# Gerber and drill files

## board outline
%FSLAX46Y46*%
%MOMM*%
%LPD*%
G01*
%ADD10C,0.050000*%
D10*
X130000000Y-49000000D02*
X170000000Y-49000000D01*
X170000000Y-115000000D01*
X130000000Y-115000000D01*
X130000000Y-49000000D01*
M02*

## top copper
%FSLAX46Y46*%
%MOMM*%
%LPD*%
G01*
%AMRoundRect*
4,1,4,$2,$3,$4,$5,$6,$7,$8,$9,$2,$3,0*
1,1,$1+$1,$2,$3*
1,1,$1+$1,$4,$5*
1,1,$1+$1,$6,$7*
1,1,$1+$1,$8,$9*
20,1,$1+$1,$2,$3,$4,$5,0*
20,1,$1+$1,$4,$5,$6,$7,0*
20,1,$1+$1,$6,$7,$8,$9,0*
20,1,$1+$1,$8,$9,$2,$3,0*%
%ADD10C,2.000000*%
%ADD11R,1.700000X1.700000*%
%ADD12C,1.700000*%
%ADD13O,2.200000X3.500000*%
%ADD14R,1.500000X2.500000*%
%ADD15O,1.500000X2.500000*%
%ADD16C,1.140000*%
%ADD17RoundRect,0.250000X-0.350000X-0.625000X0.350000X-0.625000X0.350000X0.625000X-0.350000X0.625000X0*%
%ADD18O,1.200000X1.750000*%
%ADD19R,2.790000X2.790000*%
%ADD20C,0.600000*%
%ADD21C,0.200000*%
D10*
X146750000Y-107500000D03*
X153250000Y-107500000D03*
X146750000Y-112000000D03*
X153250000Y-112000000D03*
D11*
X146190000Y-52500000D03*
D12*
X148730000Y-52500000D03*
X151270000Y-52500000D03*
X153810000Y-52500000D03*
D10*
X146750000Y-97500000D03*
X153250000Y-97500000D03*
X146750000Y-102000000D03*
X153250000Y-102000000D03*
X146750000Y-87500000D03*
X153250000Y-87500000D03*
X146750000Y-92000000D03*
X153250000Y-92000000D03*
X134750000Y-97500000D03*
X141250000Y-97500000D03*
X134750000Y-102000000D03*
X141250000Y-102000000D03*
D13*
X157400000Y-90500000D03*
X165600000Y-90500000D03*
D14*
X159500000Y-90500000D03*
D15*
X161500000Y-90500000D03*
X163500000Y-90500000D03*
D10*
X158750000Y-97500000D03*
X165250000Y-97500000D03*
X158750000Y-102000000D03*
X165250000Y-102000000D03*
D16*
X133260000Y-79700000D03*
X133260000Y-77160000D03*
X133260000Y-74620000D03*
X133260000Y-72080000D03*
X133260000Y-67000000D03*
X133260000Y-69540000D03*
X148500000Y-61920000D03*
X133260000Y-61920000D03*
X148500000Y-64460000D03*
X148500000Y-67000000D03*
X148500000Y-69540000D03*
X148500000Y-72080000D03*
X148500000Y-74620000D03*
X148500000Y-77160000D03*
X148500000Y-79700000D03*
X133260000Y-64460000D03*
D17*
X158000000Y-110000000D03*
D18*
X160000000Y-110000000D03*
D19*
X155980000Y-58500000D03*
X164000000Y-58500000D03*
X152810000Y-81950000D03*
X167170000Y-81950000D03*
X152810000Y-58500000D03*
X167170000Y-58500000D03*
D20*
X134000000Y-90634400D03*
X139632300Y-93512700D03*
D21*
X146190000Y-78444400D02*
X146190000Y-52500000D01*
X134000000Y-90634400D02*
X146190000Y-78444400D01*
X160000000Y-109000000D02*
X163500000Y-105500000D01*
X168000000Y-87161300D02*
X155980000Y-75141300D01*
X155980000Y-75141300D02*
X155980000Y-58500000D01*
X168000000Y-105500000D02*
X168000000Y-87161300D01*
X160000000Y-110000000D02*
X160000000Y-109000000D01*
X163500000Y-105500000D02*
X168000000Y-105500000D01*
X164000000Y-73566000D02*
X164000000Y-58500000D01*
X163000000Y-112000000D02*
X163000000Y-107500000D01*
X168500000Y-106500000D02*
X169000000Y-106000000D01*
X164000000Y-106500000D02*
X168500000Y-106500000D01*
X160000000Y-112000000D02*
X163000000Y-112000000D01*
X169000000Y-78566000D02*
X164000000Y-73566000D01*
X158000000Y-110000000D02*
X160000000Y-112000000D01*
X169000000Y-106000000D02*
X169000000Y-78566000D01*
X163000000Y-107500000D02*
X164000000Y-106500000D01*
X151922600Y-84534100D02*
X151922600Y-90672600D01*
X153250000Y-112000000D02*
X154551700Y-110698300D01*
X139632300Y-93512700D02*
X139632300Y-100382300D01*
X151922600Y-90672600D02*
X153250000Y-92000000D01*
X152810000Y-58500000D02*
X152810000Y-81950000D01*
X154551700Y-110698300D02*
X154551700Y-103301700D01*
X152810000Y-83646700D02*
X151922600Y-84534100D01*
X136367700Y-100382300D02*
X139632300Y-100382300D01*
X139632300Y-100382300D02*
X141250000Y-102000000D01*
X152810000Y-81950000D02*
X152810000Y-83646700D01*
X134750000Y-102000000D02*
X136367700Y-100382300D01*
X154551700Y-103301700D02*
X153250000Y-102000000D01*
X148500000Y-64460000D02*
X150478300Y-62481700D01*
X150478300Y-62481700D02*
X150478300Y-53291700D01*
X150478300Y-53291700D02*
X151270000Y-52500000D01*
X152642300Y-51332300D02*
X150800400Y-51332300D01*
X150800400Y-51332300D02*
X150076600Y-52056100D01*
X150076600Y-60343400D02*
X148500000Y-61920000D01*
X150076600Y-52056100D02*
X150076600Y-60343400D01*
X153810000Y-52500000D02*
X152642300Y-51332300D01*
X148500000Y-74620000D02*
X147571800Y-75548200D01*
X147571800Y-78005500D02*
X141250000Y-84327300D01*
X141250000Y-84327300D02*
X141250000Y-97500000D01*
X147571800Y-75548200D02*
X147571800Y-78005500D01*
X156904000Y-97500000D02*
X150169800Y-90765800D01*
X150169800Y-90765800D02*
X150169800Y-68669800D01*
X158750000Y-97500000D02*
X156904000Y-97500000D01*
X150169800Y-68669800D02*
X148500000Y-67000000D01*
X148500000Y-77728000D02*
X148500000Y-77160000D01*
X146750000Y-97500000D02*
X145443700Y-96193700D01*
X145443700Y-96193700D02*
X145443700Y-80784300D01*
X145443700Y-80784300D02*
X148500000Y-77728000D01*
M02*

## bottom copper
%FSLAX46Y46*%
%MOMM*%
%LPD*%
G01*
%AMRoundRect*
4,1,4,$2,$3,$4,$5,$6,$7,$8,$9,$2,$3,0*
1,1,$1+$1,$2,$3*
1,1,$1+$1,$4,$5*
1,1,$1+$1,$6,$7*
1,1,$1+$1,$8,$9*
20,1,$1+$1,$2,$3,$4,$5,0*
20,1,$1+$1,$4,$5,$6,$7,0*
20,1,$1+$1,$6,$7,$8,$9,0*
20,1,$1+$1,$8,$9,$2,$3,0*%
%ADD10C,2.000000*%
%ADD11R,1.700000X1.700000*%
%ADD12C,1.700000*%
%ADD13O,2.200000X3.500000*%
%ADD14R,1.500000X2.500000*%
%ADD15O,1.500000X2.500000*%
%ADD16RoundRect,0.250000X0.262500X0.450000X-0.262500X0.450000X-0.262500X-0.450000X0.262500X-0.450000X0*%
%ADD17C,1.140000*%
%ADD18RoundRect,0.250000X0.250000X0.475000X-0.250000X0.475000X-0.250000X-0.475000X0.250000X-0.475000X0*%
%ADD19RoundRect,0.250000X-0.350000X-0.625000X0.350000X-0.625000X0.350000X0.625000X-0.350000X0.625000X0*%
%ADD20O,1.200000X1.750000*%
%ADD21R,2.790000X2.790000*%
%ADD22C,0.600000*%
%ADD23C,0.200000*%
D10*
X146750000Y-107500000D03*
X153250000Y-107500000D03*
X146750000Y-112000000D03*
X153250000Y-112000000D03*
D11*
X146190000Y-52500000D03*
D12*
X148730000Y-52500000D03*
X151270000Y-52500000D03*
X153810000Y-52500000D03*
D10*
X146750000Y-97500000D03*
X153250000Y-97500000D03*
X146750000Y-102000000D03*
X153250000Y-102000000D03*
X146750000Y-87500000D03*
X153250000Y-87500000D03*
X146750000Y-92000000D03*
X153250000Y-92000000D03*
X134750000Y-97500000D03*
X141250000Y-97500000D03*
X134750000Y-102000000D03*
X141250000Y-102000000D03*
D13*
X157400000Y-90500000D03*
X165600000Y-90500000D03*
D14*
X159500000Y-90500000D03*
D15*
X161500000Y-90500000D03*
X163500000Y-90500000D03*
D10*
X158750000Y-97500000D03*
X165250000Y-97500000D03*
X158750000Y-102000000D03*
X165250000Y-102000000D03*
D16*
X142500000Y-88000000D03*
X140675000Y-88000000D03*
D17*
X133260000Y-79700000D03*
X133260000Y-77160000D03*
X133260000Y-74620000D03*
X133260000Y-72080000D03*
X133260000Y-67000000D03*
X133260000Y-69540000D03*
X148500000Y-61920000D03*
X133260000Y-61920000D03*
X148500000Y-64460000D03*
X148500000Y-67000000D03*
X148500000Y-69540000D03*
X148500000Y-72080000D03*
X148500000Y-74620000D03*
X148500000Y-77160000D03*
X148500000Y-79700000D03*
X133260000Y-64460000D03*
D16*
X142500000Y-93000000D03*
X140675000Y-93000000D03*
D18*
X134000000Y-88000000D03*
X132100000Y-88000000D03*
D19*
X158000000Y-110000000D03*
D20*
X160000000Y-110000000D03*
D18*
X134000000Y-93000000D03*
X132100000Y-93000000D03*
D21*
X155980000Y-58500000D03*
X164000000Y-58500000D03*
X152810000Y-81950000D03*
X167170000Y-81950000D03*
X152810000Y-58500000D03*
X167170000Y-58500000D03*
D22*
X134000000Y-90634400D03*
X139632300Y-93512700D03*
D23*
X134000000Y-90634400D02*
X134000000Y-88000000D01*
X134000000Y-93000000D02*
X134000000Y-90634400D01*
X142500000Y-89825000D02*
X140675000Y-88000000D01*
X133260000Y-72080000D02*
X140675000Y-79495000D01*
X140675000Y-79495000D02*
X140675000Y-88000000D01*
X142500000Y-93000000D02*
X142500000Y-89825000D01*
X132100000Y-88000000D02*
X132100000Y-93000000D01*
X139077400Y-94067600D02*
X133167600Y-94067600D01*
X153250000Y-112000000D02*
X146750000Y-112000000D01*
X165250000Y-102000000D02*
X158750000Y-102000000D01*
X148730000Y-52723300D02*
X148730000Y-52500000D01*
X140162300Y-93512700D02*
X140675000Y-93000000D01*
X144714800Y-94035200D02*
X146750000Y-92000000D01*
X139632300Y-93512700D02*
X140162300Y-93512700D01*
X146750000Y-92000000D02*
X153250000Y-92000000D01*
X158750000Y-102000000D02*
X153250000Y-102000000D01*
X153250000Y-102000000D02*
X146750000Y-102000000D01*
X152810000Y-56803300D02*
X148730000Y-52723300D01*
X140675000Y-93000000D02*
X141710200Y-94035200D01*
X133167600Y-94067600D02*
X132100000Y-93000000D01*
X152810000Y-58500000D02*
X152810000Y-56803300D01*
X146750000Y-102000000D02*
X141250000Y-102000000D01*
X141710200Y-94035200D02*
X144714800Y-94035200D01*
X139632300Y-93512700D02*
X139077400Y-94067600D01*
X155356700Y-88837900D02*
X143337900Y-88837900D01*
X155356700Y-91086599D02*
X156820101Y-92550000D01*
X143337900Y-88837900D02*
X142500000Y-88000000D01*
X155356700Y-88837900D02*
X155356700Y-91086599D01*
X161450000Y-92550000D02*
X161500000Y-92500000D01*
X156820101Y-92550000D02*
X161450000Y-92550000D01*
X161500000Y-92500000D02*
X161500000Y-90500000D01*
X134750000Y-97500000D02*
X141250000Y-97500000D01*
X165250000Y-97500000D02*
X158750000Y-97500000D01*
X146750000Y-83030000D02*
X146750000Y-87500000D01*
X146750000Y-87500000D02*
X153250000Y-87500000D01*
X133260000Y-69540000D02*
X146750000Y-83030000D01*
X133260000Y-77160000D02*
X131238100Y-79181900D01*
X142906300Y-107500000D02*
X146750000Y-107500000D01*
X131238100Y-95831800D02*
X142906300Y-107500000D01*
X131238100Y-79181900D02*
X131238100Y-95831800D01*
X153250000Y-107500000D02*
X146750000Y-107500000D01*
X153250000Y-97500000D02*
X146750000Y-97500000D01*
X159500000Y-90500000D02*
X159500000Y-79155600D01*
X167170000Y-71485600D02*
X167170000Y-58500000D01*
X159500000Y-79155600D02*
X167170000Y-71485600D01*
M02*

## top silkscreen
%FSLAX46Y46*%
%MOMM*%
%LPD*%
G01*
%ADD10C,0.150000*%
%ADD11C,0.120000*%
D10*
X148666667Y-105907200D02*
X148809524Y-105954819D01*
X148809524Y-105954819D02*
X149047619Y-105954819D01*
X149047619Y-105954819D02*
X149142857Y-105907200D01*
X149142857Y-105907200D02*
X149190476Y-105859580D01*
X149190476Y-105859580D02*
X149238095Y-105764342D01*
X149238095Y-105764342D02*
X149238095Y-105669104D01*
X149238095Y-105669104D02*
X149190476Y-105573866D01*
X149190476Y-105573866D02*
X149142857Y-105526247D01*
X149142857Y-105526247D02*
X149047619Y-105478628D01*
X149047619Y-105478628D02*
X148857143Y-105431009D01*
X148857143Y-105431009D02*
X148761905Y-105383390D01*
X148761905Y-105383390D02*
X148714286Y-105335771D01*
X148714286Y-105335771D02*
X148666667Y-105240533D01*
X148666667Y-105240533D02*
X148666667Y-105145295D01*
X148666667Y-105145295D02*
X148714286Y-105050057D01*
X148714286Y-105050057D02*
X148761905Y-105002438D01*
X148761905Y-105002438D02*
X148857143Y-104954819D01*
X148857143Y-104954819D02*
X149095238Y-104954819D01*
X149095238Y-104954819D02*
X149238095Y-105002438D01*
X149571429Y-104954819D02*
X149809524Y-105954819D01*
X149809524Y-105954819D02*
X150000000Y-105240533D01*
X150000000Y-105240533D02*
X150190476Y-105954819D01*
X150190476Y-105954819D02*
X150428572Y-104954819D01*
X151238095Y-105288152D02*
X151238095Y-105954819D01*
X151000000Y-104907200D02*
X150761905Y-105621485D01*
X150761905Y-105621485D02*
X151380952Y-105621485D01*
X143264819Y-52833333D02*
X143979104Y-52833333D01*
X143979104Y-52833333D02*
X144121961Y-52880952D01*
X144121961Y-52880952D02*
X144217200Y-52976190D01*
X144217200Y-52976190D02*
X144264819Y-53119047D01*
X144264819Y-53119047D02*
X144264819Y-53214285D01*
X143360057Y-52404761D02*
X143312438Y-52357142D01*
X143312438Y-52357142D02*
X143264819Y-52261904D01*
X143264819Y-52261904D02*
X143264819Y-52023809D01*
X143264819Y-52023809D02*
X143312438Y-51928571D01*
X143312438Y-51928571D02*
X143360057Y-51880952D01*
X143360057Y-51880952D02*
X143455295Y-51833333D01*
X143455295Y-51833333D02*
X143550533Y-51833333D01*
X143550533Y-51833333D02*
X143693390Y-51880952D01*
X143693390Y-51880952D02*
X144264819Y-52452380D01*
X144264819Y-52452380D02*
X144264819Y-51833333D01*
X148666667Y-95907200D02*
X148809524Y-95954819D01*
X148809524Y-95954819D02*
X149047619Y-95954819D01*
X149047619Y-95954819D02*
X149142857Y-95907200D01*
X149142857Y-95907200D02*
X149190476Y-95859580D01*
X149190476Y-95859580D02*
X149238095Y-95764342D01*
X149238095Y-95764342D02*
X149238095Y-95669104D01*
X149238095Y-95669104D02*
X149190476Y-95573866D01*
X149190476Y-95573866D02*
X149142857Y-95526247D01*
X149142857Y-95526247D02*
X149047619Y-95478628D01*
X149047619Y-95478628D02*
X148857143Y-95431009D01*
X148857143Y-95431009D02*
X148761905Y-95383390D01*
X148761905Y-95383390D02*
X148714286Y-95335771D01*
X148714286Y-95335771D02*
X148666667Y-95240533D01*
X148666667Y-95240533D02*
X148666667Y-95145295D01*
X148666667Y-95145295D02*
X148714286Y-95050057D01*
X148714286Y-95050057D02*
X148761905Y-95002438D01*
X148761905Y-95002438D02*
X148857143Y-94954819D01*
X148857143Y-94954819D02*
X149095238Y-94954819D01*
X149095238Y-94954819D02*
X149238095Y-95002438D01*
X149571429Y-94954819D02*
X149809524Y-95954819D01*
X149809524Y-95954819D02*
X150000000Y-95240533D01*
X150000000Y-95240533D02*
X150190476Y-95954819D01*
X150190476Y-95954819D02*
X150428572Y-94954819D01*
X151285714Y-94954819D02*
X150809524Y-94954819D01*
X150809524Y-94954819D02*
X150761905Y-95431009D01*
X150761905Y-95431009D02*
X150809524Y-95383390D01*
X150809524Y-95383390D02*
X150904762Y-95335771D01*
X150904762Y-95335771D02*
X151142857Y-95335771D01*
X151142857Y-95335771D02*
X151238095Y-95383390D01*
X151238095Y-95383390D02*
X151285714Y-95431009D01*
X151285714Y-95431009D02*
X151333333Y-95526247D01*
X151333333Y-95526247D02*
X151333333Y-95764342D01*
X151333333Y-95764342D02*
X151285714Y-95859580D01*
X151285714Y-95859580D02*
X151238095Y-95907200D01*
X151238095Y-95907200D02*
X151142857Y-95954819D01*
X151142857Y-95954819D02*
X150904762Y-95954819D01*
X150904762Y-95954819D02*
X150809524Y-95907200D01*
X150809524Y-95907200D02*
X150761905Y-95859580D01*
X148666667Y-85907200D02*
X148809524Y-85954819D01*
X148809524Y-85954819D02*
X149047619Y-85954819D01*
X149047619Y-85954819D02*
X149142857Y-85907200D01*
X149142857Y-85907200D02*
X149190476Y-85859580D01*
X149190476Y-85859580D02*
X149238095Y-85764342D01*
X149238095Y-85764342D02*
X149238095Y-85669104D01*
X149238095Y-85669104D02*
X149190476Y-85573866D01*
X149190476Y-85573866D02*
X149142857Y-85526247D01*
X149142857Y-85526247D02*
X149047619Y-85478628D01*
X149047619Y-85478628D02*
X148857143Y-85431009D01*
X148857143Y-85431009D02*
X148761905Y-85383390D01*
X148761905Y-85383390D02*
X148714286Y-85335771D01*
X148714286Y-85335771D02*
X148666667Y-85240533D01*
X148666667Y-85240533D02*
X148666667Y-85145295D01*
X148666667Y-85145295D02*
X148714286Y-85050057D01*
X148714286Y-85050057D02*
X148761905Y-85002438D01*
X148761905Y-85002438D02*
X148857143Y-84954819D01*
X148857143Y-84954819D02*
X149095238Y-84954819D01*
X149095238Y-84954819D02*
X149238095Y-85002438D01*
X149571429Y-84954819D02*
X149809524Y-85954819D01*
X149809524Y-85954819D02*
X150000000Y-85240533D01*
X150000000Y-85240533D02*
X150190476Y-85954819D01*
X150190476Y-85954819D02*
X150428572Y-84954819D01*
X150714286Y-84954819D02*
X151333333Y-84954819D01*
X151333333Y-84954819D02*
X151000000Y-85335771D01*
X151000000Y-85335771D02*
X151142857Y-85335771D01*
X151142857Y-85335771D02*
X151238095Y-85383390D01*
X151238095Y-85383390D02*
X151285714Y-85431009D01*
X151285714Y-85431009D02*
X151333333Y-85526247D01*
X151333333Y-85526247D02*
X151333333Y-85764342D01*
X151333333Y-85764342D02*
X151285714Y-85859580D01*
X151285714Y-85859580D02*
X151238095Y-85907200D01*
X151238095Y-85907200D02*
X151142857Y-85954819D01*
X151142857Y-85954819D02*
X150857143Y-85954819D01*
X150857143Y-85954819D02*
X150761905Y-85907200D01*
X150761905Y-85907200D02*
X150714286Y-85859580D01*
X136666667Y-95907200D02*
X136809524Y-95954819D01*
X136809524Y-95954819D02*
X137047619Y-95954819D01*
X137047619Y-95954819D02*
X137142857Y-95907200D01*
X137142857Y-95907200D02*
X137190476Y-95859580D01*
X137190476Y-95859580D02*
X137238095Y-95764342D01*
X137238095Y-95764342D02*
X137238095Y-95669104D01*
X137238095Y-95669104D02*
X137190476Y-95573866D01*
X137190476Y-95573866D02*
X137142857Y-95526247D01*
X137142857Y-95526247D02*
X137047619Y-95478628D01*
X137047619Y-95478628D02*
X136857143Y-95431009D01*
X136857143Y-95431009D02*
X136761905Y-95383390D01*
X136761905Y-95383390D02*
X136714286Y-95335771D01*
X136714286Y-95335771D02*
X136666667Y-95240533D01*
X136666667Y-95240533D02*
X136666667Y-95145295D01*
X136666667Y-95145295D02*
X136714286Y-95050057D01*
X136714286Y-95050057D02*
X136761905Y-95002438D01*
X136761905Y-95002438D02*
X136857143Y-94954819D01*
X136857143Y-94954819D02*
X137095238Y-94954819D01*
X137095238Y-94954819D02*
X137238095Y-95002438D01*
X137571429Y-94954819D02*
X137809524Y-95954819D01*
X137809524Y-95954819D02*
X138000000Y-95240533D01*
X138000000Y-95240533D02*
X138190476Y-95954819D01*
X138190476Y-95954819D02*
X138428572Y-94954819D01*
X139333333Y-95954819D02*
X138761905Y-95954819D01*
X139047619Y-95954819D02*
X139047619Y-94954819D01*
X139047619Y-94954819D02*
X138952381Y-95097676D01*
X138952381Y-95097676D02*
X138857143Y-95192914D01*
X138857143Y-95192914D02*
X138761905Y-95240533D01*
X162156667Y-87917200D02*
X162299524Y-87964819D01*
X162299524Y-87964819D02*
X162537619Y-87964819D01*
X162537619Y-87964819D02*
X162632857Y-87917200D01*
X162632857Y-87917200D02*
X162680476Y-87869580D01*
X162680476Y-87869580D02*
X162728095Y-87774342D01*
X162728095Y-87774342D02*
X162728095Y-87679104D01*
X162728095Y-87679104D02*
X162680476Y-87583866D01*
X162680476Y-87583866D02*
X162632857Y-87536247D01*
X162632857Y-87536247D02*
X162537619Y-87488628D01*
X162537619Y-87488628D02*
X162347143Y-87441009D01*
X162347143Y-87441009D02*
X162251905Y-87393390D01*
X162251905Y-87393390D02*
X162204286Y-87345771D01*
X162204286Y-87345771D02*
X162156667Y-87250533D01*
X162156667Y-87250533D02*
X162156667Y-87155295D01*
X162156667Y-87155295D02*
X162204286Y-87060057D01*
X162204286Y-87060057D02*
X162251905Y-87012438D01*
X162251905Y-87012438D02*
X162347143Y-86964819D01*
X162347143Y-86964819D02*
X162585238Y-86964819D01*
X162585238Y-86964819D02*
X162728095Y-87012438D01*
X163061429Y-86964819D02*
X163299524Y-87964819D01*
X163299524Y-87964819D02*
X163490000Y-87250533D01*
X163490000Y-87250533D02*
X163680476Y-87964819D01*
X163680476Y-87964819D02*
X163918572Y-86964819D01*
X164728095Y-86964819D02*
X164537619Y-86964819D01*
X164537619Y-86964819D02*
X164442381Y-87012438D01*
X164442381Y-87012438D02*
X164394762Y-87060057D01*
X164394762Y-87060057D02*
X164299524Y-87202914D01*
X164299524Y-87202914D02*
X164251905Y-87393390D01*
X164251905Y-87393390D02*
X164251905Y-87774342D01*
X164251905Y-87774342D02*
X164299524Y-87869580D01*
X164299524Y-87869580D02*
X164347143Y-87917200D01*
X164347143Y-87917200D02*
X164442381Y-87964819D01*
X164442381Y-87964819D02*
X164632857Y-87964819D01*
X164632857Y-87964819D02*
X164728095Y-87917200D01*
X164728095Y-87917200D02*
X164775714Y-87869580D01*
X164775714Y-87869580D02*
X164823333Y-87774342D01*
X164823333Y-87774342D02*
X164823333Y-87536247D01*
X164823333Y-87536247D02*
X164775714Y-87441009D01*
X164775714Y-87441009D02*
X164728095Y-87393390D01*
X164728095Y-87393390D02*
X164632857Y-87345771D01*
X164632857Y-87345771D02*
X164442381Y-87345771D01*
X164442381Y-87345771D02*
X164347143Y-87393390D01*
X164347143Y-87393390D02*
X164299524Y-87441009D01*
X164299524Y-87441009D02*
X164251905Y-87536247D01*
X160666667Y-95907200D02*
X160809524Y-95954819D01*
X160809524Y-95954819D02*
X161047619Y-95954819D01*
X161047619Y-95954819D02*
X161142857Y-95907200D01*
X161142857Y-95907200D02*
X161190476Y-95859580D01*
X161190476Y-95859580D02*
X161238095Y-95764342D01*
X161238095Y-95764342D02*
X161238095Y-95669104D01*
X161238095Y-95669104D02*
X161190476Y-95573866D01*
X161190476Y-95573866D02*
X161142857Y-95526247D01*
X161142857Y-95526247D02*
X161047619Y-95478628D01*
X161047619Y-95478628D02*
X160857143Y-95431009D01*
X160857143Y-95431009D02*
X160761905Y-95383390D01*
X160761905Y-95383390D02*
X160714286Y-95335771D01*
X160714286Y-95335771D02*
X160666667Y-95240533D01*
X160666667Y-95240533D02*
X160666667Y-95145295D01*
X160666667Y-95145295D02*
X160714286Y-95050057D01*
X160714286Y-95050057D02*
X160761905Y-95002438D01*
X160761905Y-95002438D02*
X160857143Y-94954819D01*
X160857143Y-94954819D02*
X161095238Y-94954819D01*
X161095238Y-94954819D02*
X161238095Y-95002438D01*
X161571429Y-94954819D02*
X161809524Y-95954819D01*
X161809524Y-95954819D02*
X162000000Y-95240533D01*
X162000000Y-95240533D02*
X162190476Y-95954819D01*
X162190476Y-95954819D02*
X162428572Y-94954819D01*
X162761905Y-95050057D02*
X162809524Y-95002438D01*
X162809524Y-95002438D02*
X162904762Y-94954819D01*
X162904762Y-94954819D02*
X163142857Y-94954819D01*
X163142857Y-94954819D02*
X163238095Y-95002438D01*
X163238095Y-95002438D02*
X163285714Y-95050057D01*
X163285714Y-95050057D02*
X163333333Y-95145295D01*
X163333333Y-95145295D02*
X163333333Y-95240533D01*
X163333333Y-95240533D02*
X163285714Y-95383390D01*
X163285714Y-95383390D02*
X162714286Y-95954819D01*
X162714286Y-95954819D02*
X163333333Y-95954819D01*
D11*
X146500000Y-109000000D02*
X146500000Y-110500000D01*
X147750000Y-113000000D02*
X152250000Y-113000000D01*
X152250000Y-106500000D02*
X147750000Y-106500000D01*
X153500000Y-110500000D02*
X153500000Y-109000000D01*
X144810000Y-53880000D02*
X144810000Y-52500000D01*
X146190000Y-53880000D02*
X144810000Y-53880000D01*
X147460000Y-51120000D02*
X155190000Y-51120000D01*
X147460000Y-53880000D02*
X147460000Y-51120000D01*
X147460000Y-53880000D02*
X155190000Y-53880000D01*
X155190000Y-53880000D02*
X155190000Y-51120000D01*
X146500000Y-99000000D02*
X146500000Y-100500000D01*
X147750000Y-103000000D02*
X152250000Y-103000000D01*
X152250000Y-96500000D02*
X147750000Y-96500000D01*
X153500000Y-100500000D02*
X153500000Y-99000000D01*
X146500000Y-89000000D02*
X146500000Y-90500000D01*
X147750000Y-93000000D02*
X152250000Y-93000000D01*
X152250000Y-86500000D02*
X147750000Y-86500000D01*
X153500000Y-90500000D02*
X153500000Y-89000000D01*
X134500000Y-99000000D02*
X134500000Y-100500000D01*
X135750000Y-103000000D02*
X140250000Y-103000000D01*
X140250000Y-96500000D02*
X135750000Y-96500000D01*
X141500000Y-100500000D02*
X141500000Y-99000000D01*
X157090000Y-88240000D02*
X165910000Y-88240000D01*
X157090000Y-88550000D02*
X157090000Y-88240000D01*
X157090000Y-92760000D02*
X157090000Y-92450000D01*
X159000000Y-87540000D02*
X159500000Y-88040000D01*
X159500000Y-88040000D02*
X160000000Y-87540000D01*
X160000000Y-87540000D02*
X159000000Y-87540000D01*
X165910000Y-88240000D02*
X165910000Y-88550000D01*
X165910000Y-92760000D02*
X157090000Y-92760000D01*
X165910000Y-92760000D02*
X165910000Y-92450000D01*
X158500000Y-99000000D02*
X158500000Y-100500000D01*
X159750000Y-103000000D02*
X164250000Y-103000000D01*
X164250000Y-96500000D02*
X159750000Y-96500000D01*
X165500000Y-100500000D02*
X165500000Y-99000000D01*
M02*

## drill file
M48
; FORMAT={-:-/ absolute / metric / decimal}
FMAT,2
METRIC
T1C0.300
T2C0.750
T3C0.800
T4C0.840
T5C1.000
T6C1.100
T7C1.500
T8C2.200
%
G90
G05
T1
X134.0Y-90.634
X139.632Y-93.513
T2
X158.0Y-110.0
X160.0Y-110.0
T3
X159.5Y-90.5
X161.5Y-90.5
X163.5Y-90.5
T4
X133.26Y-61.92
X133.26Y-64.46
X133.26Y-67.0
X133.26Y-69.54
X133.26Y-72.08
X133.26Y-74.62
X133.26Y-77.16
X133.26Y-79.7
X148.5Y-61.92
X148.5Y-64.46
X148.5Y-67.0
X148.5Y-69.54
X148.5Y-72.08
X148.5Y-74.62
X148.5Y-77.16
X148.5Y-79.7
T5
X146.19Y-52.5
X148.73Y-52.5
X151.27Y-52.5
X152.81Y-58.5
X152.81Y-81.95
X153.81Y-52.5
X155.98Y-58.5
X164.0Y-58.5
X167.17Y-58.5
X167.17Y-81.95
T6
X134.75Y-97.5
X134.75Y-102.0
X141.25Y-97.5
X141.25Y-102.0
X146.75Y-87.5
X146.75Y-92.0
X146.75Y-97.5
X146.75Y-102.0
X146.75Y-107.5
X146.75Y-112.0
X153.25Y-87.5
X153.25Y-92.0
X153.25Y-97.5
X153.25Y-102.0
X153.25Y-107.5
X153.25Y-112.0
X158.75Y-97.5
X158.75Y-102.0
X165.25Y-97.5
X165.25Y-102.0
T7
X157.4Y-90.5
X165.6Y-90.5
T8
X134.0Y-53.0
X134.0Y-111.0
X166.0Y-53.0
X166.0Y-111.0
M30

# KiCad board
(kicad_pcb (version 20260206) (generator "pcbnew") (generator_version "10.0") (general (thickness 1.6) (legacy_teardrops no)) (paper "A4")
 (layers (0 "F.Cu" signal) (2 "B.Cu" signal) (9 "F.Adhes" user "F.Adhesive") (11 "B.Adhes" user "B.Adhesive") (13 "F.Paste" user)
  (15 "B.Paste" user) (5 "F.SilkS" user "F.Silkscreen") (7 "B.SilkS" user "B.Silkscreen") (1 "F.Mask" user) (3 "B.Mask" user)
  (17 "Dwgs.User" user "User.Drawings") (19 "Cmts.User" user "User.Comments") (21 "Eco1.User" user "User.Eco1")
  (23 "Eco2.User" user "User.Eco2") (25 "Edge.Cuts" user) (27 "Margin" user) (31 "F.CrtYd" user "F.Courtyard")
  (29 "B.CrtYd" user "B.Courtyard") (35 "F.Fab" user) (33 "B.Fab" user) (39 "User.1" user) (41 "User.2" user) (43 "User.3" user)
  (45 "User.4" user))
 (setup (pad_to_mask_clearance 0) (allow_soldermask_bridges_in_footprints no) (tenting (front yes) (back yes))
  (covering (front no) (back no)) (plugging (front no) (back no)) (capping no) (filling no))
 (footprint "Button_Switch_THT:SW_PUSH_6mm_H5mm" (layer "F.Cu") (at 146.75 107.5)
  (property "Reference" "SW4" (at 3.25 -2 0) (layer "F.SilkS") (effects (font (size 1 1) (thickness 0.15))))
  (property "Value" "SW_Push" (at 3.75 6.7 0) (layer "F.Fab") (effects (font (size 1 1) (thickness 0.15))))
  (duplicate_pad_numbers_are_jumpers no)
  (fp_line (start -0.25 1.5) (end -0.25 3) (stroke (width 0.12) (type solid)) (layer "F.SilkS"))
  (fp_line (start 1 5.5) (end 5.5 5.5) (stroke (width 0.12) (type solid)) (layer "F.SilkS"))
  (fp_line (start 5.5 -1) (end 1 -1) (stroke (width 0.12) (type solid)) (layer "F.SilkS"))
  (fp_line (start 6.75 3) (end 6.75 1.5) (stroke (width 0.12) (type solid)) (layer "F.SilkS"))
  (pad "1" thru_hole circle (at 0 0 90) (size 2 2) (drill 1.1) (layers "*.Cu" "*.Mask") (remove_unused_layers no) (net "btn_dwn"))
  (pad "1" thru_hole circle (at 6.5 0 90) (size 2 2) (drill 1.1) (layers "*.Cu" "*.Mask") (remove_unused_layers no) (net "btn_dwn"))
  (pad "2" thru_hole circle (at 0 4.5 90) (size 2 2) (drill 1.1) (layers "*.Cu" "*.Mask") (remove_unused_layers no) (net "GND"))
  (pad "2" thru_hole circle (at 6.5 4.5 90) (size 2 2) (drill 1.1) (layers "*.Cu" "*.Mask") (remove_unused_layers no) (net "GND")))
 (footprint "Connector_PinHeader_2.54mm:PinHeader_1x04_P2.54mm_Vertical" (layer "F.Cu") (at 146.19 52.5 90)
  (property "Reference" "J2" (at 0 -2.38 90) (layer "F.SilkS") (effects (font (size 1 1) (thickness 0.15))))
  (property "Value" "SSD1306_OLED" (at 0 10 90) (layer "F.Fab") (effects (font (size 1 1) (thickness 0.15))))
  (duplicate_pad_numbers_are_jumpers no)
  (fp_line (start -1.38 -1.38) (end 0 -1.38) (stroke (width 0.12) (type solid)) (layer "F.SilkS"))
  (fp_line (start -1.38 0) (end -1.38 -1.38) (stroke (width 0.12) (type solid)) (layer "F.SilkS"))
  (fp_line (start 1.38 1.27) (end 1.38 9) (stroke (width 0.12) (type solid)) (layer "F.SilkS"))
  (fp_line (start -1.38 1.27) (end 1.38 1.27) (stroke (width 0.12) (type solid)) (layer "F.SilkS"))
  (fp_line (start -1.38 1.27) (end -1.38 9) (stroke (width 0.12) (type solid)) (layer "F.SilkS"))
  (fp_line (start -1.38 9) (end 1.38 9) (stroke (width 0.12) (type solid)) (layer "F.SilkS"))
  (pad "1" thru_hole rect (at 0 0 90) (size 1.7 1.7) (drill 1) (layers "*.Cu" "*.Mask") (remove_unused_layers no) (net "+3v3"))
  (pad "2" thru_hole circle (at 0 2.54 90) (size 1.7 1.7) (drill 1) (layers "*.Cu" "*.Mask") (remove_unused_layers no) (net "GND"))
  (pad "3" thru_hole circle (at 0 5.08 90) (size 1.7 1.7) (drill 1) (layers "*.Cu" "*.Mask") (remove_unused_layers no) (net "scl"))
  (pad "4" thru_hole circle (at 0 7.62 90) (size 1.7 1.7) (drill 1) (layers "*.Cu" "*.Mask") (remove_unused_layers no) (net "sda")))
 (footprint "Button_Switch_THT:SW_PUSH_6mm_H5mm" (layer "F.Cu") (at 146.75 97.5)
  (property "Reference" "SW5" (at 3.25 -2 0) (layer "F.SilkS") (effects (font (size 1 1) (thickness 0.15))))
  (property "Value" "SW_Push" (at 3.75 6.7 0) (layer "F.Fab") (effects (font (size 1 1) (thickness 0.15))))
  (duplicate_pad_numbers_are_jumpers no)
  (fp_line (start -0.25 1.5) (end -0.25 3) (stroke (width 0.12) (type solid)) (layer "F.SilkS"))
  (fp_line (start 1 5.5) (end 5.5 5.5) (stroke (width 0.12) (type solid)) (layer "F.SilkS"))
  (fp_line (start 5.5 -1) (end 1 -1) (stroke (width 0.12) (type solid)) (layer "F.SilkS"))
  (fp_line (start 6.75 3) (end 6.75 1.5) (stroke (width 0.12) (type solid)) (layer "F.SilkS"))
  (pad "1" thru_hole circle (at 0 0 90) (size 2 2) (drill 1.1) (layers "*.Cu" "*.Mask") (remove_unused_layers no) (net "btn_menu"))
  (pad "1" thru_hole circle (at 6.5 0 90) (size 2 2) (drill 1.1) (layers "*.Cu" "*.Mask") (remove_unused_layers no) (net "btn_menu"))
  (pad "2" thru_hole circle (at 0 4.5 90) (size 2 2) (drill 1.1) (layers "*.Cu" "*.Mask") (remove_unused_layers no) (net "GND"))
  (pad "2" thru_hole circle (at 6.5 4.5 90) (size 2 2) (drill 1.1) (layers "*.Cu" "*.Mask") (remove_unused_layers no) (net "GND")))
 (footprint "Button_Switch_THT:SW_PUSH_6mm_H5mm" (layer "F.Cu") (at 146.75 87.5)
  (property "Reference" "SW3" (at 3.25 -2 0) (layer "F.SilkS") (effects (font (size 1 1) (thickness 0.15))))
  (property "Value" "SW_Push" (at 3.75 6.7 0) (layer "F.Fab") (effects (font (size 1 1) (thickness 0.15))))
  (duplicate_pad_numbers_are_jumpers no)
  (fp_line (start -0.25 1.5) (end -0.25 3) (stroke (width 0.12) (type solid)) (layer "F.SilkS"))
  (fp_line (start 1 5.5) (end 5.5 5.5) (stroke (width 0.12) (type solid)) (layer "F.SilkS"))
  (fp_line (start 5.5 -1) (end 1 -1) (stroke (width 0.12) (type solid)) (layer "F.SilkS"))
  (fp_line (start 6.75 3) (end 6.75 1.5) (stroke (width 0.12) (type solid)) (layer "F.SilkS"))
  (pad "1" thru_hole circle (at 0 0 90) (size 2 2) (drill 1.1) (layers "*.Cu" "*.Mask") (remove_unused_layers no) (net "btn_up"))
  (pad "1" thru_hole circle (at 6.5 0 90) (size 2 2) (drill 1.1) (layers "*.Cu" "*.Mask") (remove_unused_layers no) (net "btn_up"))
  (pad "2" thru_hole circle (at 0 4.5 90) (size 2 2) (drill 1.1) (layers "*.Cu" "*.Mask") (remove_unused_layers no) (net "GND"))
  (pad "2" thru_hole circle (at 6.5 4.5 90) (size 2 2) (drill 1.1) (layers "*.Cu" "*.Mask") (remove_unused_layers no) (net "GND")))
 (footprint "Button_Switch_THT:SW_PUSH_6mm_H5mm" (layer "F.Cu") (at 134.75 97.5)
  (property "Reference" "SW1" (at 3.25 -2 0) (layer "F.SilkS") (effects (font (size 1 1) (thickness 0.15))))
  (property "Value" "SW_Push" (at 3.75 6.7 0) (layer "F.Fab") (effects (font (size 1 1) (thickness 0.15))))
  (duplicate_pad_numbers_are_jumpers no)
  (fp_line (start -0.25 1.5) (end -0.25 3) (stroke (width 0.12) (type solid)) (layer "F.SilkS"))
  (fp_line (start 1 5.5) (end 5.5 5.5) (stroke (width 0.12) (type solid)) (layer "F.SilkS"))
  (fp_line (start 5.5 -1) (end 1 -1) (stroke (width 0.12) (type solid)) (layer "F.SilkS"))
  (fp_line (start 6.75 3) (end 6.75 1.5) (stroke (width 0.12) (type solid)) (layer "F.SilkS"))
  (pad "1" thru_hole circle (at 0 0 90) (size 2 2) (drill 1.1) (layers "*.Cu" "*.Mask") (remove_unused_layers no) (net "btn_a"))
  (pad "1" thru_hole circle (at 6.5 0 90) (size 2 2) (drill 1.1) (layers "*.Cu" "*.Mask") (remove_unused_layers no) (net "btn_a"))
  (pad "2" thru_hole circle (at 0 4.5 90) (size 2 2) (drill 1.1) (layers "*.Cu" "*.Mask") (remove_unused_layers no) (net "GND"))
  (pad "2" thru_hole circle (at 6.5 4.5 90) (size 2 2) (drill 1.1) (layers "*.Cu" "*.Mask") (remove_unused_layers no) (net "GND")))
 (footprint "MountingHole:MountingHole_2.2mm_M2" (layer "F.Cu") (at 166 53)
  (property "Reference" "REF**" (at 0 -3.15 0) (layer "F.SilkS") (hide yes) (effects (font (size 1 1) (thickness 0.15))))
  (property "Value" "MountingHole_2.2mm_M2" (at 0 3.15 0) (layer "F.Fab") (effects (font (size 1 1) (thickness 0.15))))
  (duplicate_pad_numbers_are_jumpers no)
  (pad "" np_thru_hole circle (at 0 0) (size 2.2 2.2) (drill 2.2) (layers "*.Cu" "*.Mask")))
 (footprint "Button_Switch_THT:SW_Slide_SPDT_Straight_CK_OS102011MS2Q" (layer "F.Cu") (at 159.5 90.5)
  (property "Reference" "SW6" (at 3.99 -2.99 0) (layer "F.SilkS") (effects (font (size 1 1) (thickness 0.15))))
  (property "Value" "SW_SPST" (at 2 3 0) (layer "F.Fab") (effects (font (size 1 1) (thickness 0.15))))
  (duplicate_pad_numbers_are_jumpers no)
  (fp_line (start -2.41 -2.26) (end 6.41 -2.26) (stroke (width 0.12) (type solid)) (layer "F.SilkS"))
  (fp_line (start -2.41 -1.95) (end -2.41 -2.26) (stroke (width 0.12) (type solid)) (layer "F.SilkS"))
  (fp_line (start -2.41 2.26) (end -2.41 1.95) (stroke (width 0.12) (type solid)) (layer "F.SilkS"))
  (fp_line (start -0.5 -2.96) (end 0 -2.46) (stroke (width 0.12) (type solid)) (layer "F.SilkS"))
  (fp_line (start 0 -2.46) (end 0.5 -2.96) (stroke (width 0.12) (type solid)) (layer "F.SilkS"))
  (fp_line (start 0.5 -2.96) (end -0.5 -2.96) (stroke (width 0.12) (type solid)) (layer "F.SilkS"))
  (fp_line (start 6.41 -2.26) (end 6.41 -1.95) (stroke (width 0.12) (type solid)) (layer "F.SilkS"))
  (fp_line (start 6.41 2.26) (end -2.41 2.26) (stroke (width 0.12) (type solid)) (layer "F.SilkS"))
  (fp_line (start 6.41 2.26) (end 6.41 1.95) (stroke (width 0.12) (type solid)) (layer "F.SilkS"))
  (pad "" thru_hole oval (at -2.1 0) (size 2.2 3.5) (drill 1.5) (layers "*.Cu" "*.Mask") (remove_unused_layers no))
  (pad "" thru_hole oval (at 6.1 0) (size 2.2 3.5) (drill 1.5) (layers "*.Cu" "*.Mask") (remove_unused_layers no))
  (pad "1" thru_hole rect (at 0 0) (size 1.5 2.5) (drill 0.8) (layers "*.Cu" "*.Mask") (remove_unused_layers no) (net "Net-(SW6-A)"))
  (pad "2" thru_hole oval (at 2 0) (size 1.5 2.5) (drill 0.8) (layers "*.Cu" "*.Mask") (remove_unused_layers no) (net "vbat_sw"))
  (pad "3" thru_hole oval (at 4 0) (size 1.5 2.5) (drill 0.8) (layers "*.Cu" "*.Mask") (remove_unused_layers no)))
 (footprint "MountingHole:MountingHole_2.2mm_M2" (layer "F.Cu") (at 166 111)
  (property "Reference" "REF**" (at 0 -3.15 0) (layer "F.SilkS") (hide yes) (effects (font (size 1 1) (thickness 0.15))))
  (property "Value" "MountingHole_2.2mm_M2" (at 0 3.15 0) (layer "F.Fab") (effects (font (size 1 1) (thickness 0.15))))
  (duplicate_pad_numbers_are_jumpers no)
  (pad "" np_thru_hole circle (at 0 0) (size 2.2 2.2) (drill 2.2) (layers "*.Cu" "*.Mask")))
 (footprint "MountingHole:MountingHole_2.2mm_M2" (layer "F.Cu") (at 134 111)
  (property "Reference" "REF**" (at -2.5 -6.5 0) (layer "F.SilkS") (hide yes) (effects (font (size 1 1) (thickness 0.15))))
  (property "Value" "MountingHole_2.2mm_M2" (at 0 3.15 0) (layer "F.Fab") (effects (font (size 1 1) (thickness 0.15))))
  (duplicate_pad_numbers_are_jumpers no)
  (pad "" np_thru_hole circle (at 0 0) (size 2.2 2.2) (drill 2.2) (layers "*.Cu" "*.Mask")))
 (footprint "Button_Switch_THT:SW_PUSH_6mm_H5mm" (layer "F.Cu") (at 158.75 97.5)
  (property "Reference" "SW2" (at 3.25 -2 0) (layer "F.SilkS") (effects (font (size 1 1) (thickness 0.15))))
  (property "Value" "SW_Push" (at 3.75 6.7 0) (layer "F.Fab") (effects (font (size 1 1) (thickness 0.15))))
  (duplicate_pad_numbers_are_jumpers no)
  (fp_line (start -0.25 1.5) (end -0.25 3) (stroke (width 0.12) (type solid)) (layer "F.SilkS"))
  (fp_line (start 1 5.5) (end 5.5 5.5) (stroke (width 0.12) (type solid)) (layer "F.SilkS"))
  (fp_line (start 5.5 -1) (end 1 -1) (stroke (width 0.12) (type solid)) (layer "F.SilkS"))
  (fp_line (start 6.75 3) (end 6.75 1.5) (stroke (width 0.12) (type solid)) (layer "F.SilkS"))
  (pad "1" thru_hole circle (at 0 0 90) (size 2 2) (drill 1.1) (layers "*.Cu" "*.Mask") (remove_unused_layers no) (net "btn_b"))
  (pad "1" thru_hole circle (at 6.5 0 90) (size 2 2) (drill 1.1) (layers "*.Cu" "*.Mask") (remove_unused_layers no) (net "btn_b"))
  (pad "2" thru_hole circle (at 0 4.5 90) (size 2 2) (drill 1.1) (layers "*.Cu" "*.Mask") (remove_unused_layers no) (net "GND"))
  (pad "2" thru_hole circle (at 6.5 4.5 90) (size 2 2) (drill 1.1) (layers "*.Cu" "*.Mask") (remove_unused_layers no) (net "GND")))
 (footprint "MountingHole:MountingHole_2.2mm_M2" (layer "F.Cu") (at 134 53)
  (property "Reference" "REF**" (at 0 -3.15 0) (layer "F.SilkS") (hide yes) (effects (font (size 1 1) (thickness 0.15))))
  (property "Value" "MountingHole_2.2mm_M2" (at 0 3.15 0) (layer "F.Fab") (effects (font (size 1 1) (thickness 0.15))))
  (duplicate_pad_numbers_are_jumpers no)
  (pad "" np_thru_hole circle (at 0 0) (size 2.2 2.2) (drill 2.2) (layers "*.Cu" "*.Mask")))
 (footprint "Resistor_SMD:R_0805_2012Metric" (layer "B.Cu") (at 141.5875 88 180)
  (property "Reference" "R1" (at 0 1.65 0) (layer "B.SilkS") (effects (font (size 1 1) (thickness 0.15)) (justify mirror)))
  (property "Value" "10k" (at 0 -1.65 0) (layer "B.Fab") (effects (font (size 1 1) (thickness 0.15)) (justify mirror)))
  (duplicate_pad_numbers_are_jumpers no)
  (pad "1" smd roundrect (at -0.9125 0 180) (size 1.025 1.4) (layers "B.Cu" "B.Mask" "B.Paste") (roundrect_rratio 0.243902) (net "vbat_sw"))
  (pad "2" smd roundrect (at 0.9125 0 180) (size 1.025 1.4) (layers "B.Cu" "B.Mask" "B.Paste") (roundrect_rratio 0.243902)
   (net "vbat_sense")))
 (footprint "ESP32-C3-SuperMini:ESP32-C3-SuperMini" (layer "B.Cu") (at 140.88 70.81 180)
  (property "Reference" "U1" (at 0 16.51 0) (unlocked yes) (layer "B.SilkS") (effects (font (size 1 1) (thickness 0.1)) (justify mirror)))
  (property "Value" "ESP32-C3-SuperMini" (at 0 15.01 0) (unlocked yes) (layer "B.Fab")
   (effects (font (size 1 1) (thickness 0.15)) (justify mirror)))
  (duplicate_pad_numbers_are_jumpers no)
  (pad "0" thru_hole circle (at 7.62 -8.89 180) (size 1.14 1.14) (drill 0.84) (layers "*.Cu" "*.Mask") (remove_unused_layers no)
   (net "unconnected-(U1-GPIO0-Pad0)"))
  (pad "1" thru_hole circle (at 7.62 -6.35 180) (size 1.14 1.14) (drill 0.84) (layers "*.Cu" "*.Mask") (remove_unused_layers no)
   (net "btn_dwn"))
  (pad "2" thru_hole circle (at 7.62 -3.81 180) (size 1.14 1.14) (drill 0.84) (layers "*.Cu" "*.Mask") (remove_unused_layers no)
   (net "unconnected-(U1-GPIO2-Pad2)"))
  (pad "3" thru_hole circle (at 7.62 -1.27 180) (size 1.14 1.14) (drill 0.84) (layers "*.Cu" "*.Mask") (remove_unused_layers no)
   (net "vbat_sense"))
  (pad "3V3" thru_hole circle (at 7.62 3.81 180) (size 1.14 1.14) (drill 0.84) (layers "*.Cu" "*.Mask") (remove_unused_layers no))
  (pad "4" thru_hole circle (at 7.62 1.27 180) (size 1.14 1.14) (drill 0.84) (layers "*.Cu" "*.Mask") (remove_unused_layers no)
   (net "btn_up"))
  (pad "5" thru_hole circle (at -7.62 8.89 180) (size 1.14 1.14) (drill 0.84) (layers "*.Cu" "*.Mask") (remove_unused_layers no) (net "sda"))
  (pad "5V" thru_hole circle (at 7.62 8.89 180) (size 1.14 1.14) (drill 0.84) (layers "*.Cu" "*.Mask") (remove_unused_layers no))
  (pad "6" thru_hole circle (at -7.62 6.35 180) (size 1.14 1.14) (drill 0.84) (layers "*.Cu" "*.Mask") (remove_unused_layers no) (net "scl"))
  (pad "7" thru_hole circle (at -7.62 3.81 180) (size 1.14 1.14) (drill 0.84) (layers "*.Cu" "*.Mask") (remove_unused_layers no)
   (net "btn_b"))
  (pad "8" thru_hole circle (at -7.62 1.27 180) (size 1.14 1.14) (drill 0.84) (layers "*.Cu" "*.Mask") (remove_unused_layers no)
   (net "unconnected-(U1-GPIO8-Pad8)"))
  (pad "9" thru_hole circle (at -7.62 -1.27 180) (size 1.14 1.14) (drill 0.84) (layers "*.Cu" "*.Mask") (remove_unused_layers no)
   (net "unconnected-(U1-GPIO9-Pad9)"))
  (pad "10" thru_hole circle (at -7.62 -3.81 180) (size 1.14 1.14) (drill 0.84) (layers "*.Cu" "*.Mask") (remove_unused_layers no)
   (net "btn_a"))
  (pad "20" thru_hole circle (at -7.62 -6.35 180) (size 1.14 1.14) (drill 0.84) (layers "*.Cu" "*.Mask") (remove_unused_layers no)
   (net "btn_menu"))
  (pad "21" thru_hole circle (at -7.62 -8.89 180) (size 1.14 1.14) (drill 0.84) (layers "*.Cu" "*.Mask") (remove_unused_layers no)
   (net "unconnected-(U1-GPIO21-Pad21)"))
  (pad "GND" thru_hole circle (at 7.62 6.35 180) (size 1.14 1.14) (drill 0.84) (layers "*.Cu" "*.Mask") (remove_unused_layers no)))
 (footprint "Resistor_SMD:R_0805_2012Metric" (layer "B.Cu") (at 141.5875 93 180)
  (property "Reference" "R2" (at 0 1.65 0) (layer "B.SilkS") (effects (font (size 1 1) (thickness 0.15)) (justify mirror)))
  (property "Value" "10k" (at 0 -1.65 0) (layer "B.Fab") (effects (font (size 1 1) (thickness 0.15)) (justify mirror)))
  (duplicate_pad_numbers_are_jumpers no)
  (pad "1" smd roundrect (at -0.9125 0 180) (size 1.025 1.4) (layers "B.Cu" "B.Mask" "B.Paste") (roundrect_rratio 0.243902)
   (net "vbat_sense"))
  (pad "2" smd roundrect (at 0.9125 0 180) (size 1.025 1.4) (layers "B.Cu" "B.Mask" "B.Paste") (roundrect_rratio 0.243902) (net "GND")))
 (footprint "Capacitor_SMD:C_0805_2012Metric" (layer "B.Cu") (at 133.05 88 180)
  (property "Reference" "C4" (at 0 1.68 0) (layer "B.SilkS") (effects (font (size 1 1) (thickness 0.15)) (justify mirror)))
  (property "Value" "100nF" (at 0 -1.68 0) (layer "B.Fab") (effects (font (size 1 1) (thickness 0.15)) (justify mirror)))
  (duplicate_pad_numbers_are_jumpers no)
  (pad "1" smd roundrect (at -0.95 0 180) (size 1 1.45) (layers "B.Cu" "B.Mask" "B.Paste") (roundrect_rratio 0.25) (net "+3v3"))
  (pad "2" smd roundrect (at 0.95 0 180) (size 1 1.45) (layers "B.Cu" "B.Mask" "B.Paste") (roundrect_rratio 0.25) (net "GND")))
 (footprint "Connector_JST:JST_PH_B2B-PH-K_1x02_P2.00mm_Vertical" (layer "B.Cu") (at 158 110)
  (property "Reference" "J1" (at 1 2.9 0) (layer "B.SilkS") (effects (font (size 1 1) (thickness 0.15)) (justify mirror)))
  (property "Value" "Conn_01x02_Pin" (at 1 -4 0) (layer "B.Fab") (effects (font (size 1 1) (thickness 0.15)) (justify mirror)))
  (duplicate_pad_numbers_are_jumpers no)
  (pad "1" thru_hole roundrect (at 0 0) (size 1.2 1.75) (drill 0.75) (layers "*.Cu" "*.Mask") (remove_unused_layers no)
   (roundrect_rratio 0.208333) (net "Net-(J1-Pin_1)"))
  (pad "2" thru_hole oval (at 2 0) (size 1.2 1.75) (drill 0.75) (layers "*.Cu" "*.Mask") (remove_unused_layers no) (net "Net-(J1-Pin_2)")))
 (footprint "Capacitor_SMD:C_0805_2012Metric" (layer "B.Cu") (at 133.05 93 180)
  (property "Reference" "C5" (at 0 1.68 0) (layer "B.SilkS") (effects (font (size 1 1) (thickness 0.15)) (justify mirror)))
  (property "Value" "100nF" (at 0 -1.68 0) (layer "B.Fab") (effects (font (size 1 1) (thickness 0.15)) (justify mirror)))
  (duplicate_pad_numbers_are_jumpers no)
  (pad "1" smd roundrect (at -0.95 0 180) (size 1 1.45) (layers "B.Cu" "B.Mask" "B.Paste") (roundrect_rratio 0.25) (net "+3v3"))
  (pad "2" smd roundrect (at 0.95 0 180) (size 1 1.45) (layers "B.Cu" "B.Mask" "B.Paste") (roundrect_rratio 0.25) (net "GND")))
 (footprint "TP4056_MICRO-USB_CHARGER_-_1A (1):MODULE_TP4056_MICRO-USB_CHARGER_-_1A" (layer "B.Cu") (at 159.99 70.225 90)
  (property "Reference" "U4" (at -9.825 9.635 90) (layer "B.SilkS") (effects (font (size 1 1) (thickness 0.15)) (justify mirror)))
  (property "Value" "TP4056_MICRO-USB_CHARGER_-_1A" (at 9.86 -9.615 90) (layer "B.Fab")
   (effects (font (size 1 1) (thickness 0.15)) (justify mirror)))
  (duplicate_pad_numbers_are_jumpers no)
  (pad "BAT_N" thru_hole rect (at 11.725 -4.01 90) (size 2.79 2.79) (drill 1) (layers "*.Cu" "*.Mask") (remove_unused_layers no)
   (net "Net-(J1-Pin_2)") (solder_mask_margin 0.102))
  (pad "BAT_P" thru_hole rect (at 11.725 4.01 90) (size 2.79 2.79) (drill 1) (layers "*.Cu" "*.Mask") (remove_unused_layers no)
   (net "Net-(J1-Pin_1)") (solder_mask_margin 0.102))
  (pad "IN_N" thru_hole rect (at -11.725 -7.18 90) (size 2.79 2.79) (drill 1) (layers "*.Cu" "*.Mask") (remove_unused_layers no) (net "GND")
   (solder_mask_margin 0.102))
  (pad "IN_P" thru_hole rect (at -11.725 7.18 90) (size 2.79 2.79) (drill 1) (layers "*.Cu" "*.Mask") (remove_unused_layers no) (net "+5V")
   (solder_mask_margin 0.102))
  (pad "OUT_N" thru_hole rect (at 11.725 -7.18 90) (size 2.79 2.79) (drill 1) (layers "*.Cu" "*.Mask") (remove_unused_layers no) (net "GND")
   (solder_mask_margin 0.102))
  (pad "OUT_P" thru_hole rect (at 11.725 7.18 90) (size 2.79 2.79) (drill 1) (layers "*.Cu" "*.Mask") (remove_unused_layers no)
   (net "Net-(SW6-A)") (solder_mask_margin 0.102)))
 (gr_rect (start 130 49) (end 170 115) (stroke (width 0.05) (type solid)) (fill no) (layer "Edge.Cuts"))
 (segment (start 146.19 78.4444) (end 146.19 52.5) (width 0.2) (layer "F.Cu") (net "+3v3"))
 (segment (start 134 90.6344) (end 146.19 78.4444) (width 0.2) (layer "F.Cu") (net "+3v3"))
 (via (at 134 90.6344) (size 0.6) (drill 0.3) (layers "F.Cu" "B.Cu") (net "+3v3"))
 (segment (start 134 90.6344) (end 134 88) (width 0.2) (layer "B.Cu") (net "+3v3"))
 (segment (start 134 93) (end 134 90.6344) (width 0.2) (layer "B.Cu") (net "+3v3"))
 (segment (start 160 109) (end 163.5 105.5) (width 0.2) (layer "F.Cu") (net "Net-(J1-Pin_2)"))
 (segment (start 168 87.1613) (end 155.98 75.1413) (width 0.2) (layer "F.Cu") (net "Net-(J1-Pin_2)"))
 (segment (start 155.98 75.1413) (end 155.98 58.5) (width 0.2) (layer "F.Cu") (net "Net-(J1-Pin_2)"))
 (segment (start 168 105.5) (end 168 87.1613) (width 0.2) (layer "F.Cu") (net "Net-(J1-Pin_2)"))
 (segment (start 160 110) (end 160 109) (width 0.2) (layer "F.Cu") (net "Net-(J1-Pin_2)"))
 (segment (start 163.5 105.5) (end 168 105.5) (width 0.2) (layer "F.Cu") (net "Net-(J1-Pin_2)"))
 (segment (start 164 73.566) (end 164 58.5) (width 0.2) (layer "F.Cu") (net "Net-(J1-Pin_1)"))
 (segment (start 163 112) (end 163 107.5) (width 0.2) (layer "F.Cu") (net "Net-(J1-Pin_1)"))
 (segment (start 168.5 106.5) (end 169 106) (width 0.2) (layer "F.Cu") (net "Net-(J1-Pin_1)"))
 (segment (start 164 106.5) (end 168.5 106.5) (width 0.2) (layer "F.Cu") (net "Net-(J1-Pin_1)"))
 (segment (start 160 112) (end 163 112) (width 0.2) (layer "F.Cu") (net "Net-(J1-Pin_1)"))
 (segment (start 169 78.566) (end 164 73.566) (width 0.2) (layer "F.Cu") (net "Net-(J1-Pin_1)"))
 (segment (start 158 110) (end 160 112) (width 0.2) (layer "F.Cu") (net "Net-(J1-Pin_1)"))
 (segment (start 169 106) (end 169 78.566) (width 0.2) (layer "F.Cu") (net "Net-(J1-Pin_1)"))
 (segment (start 163 107.5) (end 164 106.5) (width 0.2) (layer "F.Cu") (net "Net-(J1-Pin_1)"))
 (segment (start 142.5 89.825) (end 140.675 88) (width 0.2) (layer "B.Cu") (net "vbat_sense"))
 (segment (start 133.26 72.08) (end 140.675 79.495) (width 0.2) (layer "B.Cu") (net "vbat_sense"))
 (segment (start 140.675 79.495) (end 140.675 88) (width 0.2) (layer "B.Cu") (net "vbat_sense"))
 (segment (start 142.5 93) (end 142.5 89.825) (width 0.2) (layer "B.Cu") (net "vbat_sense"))
 (segment (start 151.9226 84.5341) (end 151.9226 90.6726) (width 0.2) (layer "F.Cu") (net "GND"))
 (segment (start 153.25 112) (end 154.5517 110.6983) (width 0.2) (layer "F.Cu") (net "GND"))
 (segment (start 139.6323 93.5127) (end 139.6323 100.3823) (width 0.2) (layer "F.Cu") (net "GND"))
 (segment (start 151.9226 90.6726) (end 153.25 92) (width 0.2) (layer "F.Cu") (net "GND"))
 (segment (start 152.81 58.5) (end 152.81 81.95) (width 0.2) (layer "F.Cu") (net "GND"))
 (segment (start 154.5517 110.6983) (end 154.5517 103.3017) (width 0.2) (layer "F.Cu") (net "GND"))
 (segment (start 152.81 83.6467) (end 151.9226 84.5341) (width 0.2) (layer "F.Cu") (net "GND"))
 (segment (start 136.3677 100.3823) (end 139.6323 100.3823) (width 0.2) (layer "F.Cu") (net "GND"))
 (segment (start 139.6323 100.3823) (end 141.25 102) (width 0.2) (layer "F.Cu") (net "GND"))
 (segment (start 152.81 81.95) (end 152.81 83.6467) (width 0.2) (layer "F.Cu") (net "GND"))
 (segment (start 134.75 102) (end 136.3677 100.3823) (width 0.2) (layer "F.Cu") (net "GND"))
 (segment (start 154.5517 103.3017) (end 153.25 102) (width 0.2) (layer "F.Cu") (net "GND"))
 (via (at 139.6323 93.5127) (size 0.6) (drill 0.3) (layers "F.Cu" "B.Cu") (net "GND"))
 (segment (start 132.1 88) (end 132.1 93) (width 0.2) (layer "B.Cu") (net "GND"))
 (segment (start 139.0774 94.0676) (end 133.1676 94.0676) (width 0.2) (layer "B.Cu") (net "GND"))
 (segment (start 153.25 112) (end 146.75 112) (width 0.2) (layer "B.Cu") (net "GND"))
 (segment (start 165.25 102) (end 158.75 102) (width 0.2) (layer "B.Cu") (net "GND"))
 (segment (start 148.73 52.7233) (end 148.73 52.5) (width 0.2) (layer "B.Cu") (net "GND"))
 (segment (start 140.1623 93.5127) (end 140.675 93) (width 0.2) (layer "B.Cu") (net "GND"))
 (segment (start 144.7148 94.0352) (end 146.75 92) (width 0.2) (layer "B.Cu") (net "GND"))
 (segment (start 139.6323 93.5127) (end 140.1623 93.5127) (width 0.2) (layer "B.Cu") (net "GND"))
 (segment (start 146.75 92) (end 153.25 92) (width 0.2) (layer "B.Cu") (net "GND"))
 (segment (start 158.75 102) (end 153.25 102) (width 0.2) (layer "B.Cu") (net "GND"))
 (segment (start 153.25 102) (end 146.75 102) (width 0.2) (layer "B.Cu") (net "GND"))
 (segment (start 152.81 56.8033) (end 148.73 52.7233) (width 0.2) (layer "B.Cu") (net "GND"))
 (segment (start 140.675 93) (end 141.7102 94.0352) (width 0.2) (layer "B.Cu") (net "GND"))
 (segment (start 133.1676 94.0676) (end 132.1 93) (width 0.2) (layer "B.Cu") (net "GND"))
 (segment (start 152.81 58.5) (end 152.81 56.8033) (width 0.2) (layer "B.Cu") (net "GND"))
 (segment (start 146.75 102) (end 141.25 102) (width 0.2) (layer "B.Cu") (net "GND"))
 (segment (start 141.7102 94.0352) (end 144.7148 94.0352) (width 0.2) (layer "B.Cu") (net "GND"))
 (segment (start 139.6323 93.5127) (end 139.0774 94.0676) (width 0.2) (layer "B.Cu") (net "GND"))
 (segment (start 148.5 64.46) (end 150.4783 62.4817) (width 0.2) (layer "F.Cu") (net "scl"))
 (segment (start 150.4783 62.4817) (end 150.4783 53.2917) (width 0.2) (layer "F.Cu") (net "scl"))
 (segment (start 150.4783 53.2917) (end 151.27 52.5) (width 0.2) (layer "F.Cu") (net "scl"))
 (segment (start 152.6423 51.3323) (end 150.8004 51.3323) (width 0.2) (layer "F.Cu") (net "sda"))
 (segment (start 150.8004 51.3323) (end 150.0766 52.0561) (width 0.2) (layer "F.Cu") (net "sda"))
 (segment (start 150.0766 60.3434) (end 148.5 61.92) (width 0.2) (layer "F.Cu") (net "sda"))
 (segment (start 150.0766 52.0561) (end 150.0766 60.3434) (width 0.2) (layer "F.Cu") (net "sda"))
 (segment (start 153.81 52.5) (end 152.6423 51.3323) (width 0.2) (layer "F.Cu") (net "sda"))
 (segment (start 155.3567 88.8379) (end 143.3379 88.8379) (width 0.2) (layer "B.Cu") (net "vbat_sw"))
 (segment (start 155.3567 91.086599) (end 156.820101 92.55) (width 0.2) (layer "B.Cu") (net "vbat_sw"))
 (segment (start 143.3379 88.8379) (end 142.5 88) (width 0.2) (layer "B.Cu") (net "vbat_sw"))
 (segment (start 155.3567 88.8379) (end 155.3567 91.086599) (width 0.2) (layer "B.Cu") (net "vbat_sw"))
 (segment (start 161.45 92.55) (end 161.5 92.5) (width 0.2) (layer "B.Cu") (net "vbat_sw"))
 (segment (start 156.820101 92.55) (end 161.45 92.55) (width 0.2) (layer "B.Cu") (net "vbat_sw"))
 (segment (start 161.5 92.5) (end 161.5 90.5) (width 0.2) (layer "B.Cu") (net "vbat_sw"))
 (segment (start 148.5 74.62) (end 147.5718 75.5482) (width 0.2) (layer "F.Cu") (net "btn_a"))
 (segment (start 147.5718 78.0055) (end 141.25 84.3273) (width 0.2) (layer "F.Cu") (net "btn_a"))
 (segment (start 141.25 84.3273) (end 141.25 97.5) (width 0.2) (layer "F.Cu") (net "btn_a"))
 (segment (start 147.5718 75.5482) (end 147.5718 78.0055) (width 0.2) (layer "F.Cu") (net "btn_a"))
 (segment (start 134.75 97.5) (end 141.25 97.5) (width 0.2) (layer "B.Cu") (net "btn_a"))
 (segment (start 156.904 97.5) (end 150.1698 90.7658) (width 0.2) (layer "F.Cu") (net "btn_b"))
 (segment (start 150.1698 90.7658) (end 150.1698 68.6698) (width 0.2) (layer "F.Cu") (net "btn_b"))
 (segment (start 158.75 97.5) (end 156.904 97.5) (width 0.2) (layer "F.Cu") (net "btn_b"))
 (segment (start 150.1698 68.6698) (end 148.5 67) (width 0.2) (layer "F.Cu") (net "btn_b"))
 (segment (start 165.25 97.5) (end 158.75 97.5) (width 0.2) (layer "B.Cu") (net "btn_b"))
 (segment (start 146.75 83.03) (end 146.75 87.5) (width 0.2) (layer "B.Cu") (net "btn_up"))
 (segment (start 146.75 87.5) (end 153.25 87.5) (width 0.2) (layer "B.Cu") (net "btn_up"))
 (segment (start 133.26 69.54) (end 146.75 83.03) (width 0.2) (layer "B.Cu") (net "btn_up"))
 (segment (start 133.26 77.16) (end 131.2381 79.1819) (width 0.2) (layer "B.Cu") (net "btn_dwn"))
 (segment (start 142.9063 107.5) (end 146.75 107.5) (width 0.2) (layer "B.Cu") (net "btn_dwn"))
 (segment (start 131.2381 95.8318) (end 142.9063 107.5) (width 0.2) (layer "B.Cu") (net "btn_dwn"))
 (segment (start 131.2381 79.1819) (end 131.2381 95.8318) (width 0.2) (layer "B.Cu") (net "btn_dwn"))
 (segment (start 153.25 107.5) (end 146.75 107.5) (width 0.2) (layer "B.Cu") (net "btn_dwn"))
 (segment (start 148.5 77.728) (end 148.5 77.16) (width 0.2) (layer "F.Cu") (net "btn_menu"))
 (segment (start 146.75 97.5) (end 145.4437 96.1937) (width 0.2) (layer "F.Cu") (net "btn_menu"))
 (segment (start 145.4437 96.1937) (end 145.4437 80.7843) (width 0.2) (layer "F.Cu") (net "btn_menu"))
 (segment (start 145.4437 80.7843) (end 148.5 77.728) (width 0.2) (layer "F.Cu") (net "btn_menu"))
 (segment (start 153.25 97.5) (end 146.75 97.5) (width 0.2) (layer "B.Cu") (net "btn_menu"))
 (segment (start 159.5 90.5) (end 159.5 79.1556) (width 0.2) (layer "B.Cu") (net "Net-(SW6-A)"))
 (segment (start 167.17 71.4856) (end 167.17 58.5) (width 0.2) (layer "B.Cu") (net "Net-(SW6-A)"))
 (segment (start 159.5 79.1556) (end 167.17 71.4856) (width 0.2) (layer "B.Cu") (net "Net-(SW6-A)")))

